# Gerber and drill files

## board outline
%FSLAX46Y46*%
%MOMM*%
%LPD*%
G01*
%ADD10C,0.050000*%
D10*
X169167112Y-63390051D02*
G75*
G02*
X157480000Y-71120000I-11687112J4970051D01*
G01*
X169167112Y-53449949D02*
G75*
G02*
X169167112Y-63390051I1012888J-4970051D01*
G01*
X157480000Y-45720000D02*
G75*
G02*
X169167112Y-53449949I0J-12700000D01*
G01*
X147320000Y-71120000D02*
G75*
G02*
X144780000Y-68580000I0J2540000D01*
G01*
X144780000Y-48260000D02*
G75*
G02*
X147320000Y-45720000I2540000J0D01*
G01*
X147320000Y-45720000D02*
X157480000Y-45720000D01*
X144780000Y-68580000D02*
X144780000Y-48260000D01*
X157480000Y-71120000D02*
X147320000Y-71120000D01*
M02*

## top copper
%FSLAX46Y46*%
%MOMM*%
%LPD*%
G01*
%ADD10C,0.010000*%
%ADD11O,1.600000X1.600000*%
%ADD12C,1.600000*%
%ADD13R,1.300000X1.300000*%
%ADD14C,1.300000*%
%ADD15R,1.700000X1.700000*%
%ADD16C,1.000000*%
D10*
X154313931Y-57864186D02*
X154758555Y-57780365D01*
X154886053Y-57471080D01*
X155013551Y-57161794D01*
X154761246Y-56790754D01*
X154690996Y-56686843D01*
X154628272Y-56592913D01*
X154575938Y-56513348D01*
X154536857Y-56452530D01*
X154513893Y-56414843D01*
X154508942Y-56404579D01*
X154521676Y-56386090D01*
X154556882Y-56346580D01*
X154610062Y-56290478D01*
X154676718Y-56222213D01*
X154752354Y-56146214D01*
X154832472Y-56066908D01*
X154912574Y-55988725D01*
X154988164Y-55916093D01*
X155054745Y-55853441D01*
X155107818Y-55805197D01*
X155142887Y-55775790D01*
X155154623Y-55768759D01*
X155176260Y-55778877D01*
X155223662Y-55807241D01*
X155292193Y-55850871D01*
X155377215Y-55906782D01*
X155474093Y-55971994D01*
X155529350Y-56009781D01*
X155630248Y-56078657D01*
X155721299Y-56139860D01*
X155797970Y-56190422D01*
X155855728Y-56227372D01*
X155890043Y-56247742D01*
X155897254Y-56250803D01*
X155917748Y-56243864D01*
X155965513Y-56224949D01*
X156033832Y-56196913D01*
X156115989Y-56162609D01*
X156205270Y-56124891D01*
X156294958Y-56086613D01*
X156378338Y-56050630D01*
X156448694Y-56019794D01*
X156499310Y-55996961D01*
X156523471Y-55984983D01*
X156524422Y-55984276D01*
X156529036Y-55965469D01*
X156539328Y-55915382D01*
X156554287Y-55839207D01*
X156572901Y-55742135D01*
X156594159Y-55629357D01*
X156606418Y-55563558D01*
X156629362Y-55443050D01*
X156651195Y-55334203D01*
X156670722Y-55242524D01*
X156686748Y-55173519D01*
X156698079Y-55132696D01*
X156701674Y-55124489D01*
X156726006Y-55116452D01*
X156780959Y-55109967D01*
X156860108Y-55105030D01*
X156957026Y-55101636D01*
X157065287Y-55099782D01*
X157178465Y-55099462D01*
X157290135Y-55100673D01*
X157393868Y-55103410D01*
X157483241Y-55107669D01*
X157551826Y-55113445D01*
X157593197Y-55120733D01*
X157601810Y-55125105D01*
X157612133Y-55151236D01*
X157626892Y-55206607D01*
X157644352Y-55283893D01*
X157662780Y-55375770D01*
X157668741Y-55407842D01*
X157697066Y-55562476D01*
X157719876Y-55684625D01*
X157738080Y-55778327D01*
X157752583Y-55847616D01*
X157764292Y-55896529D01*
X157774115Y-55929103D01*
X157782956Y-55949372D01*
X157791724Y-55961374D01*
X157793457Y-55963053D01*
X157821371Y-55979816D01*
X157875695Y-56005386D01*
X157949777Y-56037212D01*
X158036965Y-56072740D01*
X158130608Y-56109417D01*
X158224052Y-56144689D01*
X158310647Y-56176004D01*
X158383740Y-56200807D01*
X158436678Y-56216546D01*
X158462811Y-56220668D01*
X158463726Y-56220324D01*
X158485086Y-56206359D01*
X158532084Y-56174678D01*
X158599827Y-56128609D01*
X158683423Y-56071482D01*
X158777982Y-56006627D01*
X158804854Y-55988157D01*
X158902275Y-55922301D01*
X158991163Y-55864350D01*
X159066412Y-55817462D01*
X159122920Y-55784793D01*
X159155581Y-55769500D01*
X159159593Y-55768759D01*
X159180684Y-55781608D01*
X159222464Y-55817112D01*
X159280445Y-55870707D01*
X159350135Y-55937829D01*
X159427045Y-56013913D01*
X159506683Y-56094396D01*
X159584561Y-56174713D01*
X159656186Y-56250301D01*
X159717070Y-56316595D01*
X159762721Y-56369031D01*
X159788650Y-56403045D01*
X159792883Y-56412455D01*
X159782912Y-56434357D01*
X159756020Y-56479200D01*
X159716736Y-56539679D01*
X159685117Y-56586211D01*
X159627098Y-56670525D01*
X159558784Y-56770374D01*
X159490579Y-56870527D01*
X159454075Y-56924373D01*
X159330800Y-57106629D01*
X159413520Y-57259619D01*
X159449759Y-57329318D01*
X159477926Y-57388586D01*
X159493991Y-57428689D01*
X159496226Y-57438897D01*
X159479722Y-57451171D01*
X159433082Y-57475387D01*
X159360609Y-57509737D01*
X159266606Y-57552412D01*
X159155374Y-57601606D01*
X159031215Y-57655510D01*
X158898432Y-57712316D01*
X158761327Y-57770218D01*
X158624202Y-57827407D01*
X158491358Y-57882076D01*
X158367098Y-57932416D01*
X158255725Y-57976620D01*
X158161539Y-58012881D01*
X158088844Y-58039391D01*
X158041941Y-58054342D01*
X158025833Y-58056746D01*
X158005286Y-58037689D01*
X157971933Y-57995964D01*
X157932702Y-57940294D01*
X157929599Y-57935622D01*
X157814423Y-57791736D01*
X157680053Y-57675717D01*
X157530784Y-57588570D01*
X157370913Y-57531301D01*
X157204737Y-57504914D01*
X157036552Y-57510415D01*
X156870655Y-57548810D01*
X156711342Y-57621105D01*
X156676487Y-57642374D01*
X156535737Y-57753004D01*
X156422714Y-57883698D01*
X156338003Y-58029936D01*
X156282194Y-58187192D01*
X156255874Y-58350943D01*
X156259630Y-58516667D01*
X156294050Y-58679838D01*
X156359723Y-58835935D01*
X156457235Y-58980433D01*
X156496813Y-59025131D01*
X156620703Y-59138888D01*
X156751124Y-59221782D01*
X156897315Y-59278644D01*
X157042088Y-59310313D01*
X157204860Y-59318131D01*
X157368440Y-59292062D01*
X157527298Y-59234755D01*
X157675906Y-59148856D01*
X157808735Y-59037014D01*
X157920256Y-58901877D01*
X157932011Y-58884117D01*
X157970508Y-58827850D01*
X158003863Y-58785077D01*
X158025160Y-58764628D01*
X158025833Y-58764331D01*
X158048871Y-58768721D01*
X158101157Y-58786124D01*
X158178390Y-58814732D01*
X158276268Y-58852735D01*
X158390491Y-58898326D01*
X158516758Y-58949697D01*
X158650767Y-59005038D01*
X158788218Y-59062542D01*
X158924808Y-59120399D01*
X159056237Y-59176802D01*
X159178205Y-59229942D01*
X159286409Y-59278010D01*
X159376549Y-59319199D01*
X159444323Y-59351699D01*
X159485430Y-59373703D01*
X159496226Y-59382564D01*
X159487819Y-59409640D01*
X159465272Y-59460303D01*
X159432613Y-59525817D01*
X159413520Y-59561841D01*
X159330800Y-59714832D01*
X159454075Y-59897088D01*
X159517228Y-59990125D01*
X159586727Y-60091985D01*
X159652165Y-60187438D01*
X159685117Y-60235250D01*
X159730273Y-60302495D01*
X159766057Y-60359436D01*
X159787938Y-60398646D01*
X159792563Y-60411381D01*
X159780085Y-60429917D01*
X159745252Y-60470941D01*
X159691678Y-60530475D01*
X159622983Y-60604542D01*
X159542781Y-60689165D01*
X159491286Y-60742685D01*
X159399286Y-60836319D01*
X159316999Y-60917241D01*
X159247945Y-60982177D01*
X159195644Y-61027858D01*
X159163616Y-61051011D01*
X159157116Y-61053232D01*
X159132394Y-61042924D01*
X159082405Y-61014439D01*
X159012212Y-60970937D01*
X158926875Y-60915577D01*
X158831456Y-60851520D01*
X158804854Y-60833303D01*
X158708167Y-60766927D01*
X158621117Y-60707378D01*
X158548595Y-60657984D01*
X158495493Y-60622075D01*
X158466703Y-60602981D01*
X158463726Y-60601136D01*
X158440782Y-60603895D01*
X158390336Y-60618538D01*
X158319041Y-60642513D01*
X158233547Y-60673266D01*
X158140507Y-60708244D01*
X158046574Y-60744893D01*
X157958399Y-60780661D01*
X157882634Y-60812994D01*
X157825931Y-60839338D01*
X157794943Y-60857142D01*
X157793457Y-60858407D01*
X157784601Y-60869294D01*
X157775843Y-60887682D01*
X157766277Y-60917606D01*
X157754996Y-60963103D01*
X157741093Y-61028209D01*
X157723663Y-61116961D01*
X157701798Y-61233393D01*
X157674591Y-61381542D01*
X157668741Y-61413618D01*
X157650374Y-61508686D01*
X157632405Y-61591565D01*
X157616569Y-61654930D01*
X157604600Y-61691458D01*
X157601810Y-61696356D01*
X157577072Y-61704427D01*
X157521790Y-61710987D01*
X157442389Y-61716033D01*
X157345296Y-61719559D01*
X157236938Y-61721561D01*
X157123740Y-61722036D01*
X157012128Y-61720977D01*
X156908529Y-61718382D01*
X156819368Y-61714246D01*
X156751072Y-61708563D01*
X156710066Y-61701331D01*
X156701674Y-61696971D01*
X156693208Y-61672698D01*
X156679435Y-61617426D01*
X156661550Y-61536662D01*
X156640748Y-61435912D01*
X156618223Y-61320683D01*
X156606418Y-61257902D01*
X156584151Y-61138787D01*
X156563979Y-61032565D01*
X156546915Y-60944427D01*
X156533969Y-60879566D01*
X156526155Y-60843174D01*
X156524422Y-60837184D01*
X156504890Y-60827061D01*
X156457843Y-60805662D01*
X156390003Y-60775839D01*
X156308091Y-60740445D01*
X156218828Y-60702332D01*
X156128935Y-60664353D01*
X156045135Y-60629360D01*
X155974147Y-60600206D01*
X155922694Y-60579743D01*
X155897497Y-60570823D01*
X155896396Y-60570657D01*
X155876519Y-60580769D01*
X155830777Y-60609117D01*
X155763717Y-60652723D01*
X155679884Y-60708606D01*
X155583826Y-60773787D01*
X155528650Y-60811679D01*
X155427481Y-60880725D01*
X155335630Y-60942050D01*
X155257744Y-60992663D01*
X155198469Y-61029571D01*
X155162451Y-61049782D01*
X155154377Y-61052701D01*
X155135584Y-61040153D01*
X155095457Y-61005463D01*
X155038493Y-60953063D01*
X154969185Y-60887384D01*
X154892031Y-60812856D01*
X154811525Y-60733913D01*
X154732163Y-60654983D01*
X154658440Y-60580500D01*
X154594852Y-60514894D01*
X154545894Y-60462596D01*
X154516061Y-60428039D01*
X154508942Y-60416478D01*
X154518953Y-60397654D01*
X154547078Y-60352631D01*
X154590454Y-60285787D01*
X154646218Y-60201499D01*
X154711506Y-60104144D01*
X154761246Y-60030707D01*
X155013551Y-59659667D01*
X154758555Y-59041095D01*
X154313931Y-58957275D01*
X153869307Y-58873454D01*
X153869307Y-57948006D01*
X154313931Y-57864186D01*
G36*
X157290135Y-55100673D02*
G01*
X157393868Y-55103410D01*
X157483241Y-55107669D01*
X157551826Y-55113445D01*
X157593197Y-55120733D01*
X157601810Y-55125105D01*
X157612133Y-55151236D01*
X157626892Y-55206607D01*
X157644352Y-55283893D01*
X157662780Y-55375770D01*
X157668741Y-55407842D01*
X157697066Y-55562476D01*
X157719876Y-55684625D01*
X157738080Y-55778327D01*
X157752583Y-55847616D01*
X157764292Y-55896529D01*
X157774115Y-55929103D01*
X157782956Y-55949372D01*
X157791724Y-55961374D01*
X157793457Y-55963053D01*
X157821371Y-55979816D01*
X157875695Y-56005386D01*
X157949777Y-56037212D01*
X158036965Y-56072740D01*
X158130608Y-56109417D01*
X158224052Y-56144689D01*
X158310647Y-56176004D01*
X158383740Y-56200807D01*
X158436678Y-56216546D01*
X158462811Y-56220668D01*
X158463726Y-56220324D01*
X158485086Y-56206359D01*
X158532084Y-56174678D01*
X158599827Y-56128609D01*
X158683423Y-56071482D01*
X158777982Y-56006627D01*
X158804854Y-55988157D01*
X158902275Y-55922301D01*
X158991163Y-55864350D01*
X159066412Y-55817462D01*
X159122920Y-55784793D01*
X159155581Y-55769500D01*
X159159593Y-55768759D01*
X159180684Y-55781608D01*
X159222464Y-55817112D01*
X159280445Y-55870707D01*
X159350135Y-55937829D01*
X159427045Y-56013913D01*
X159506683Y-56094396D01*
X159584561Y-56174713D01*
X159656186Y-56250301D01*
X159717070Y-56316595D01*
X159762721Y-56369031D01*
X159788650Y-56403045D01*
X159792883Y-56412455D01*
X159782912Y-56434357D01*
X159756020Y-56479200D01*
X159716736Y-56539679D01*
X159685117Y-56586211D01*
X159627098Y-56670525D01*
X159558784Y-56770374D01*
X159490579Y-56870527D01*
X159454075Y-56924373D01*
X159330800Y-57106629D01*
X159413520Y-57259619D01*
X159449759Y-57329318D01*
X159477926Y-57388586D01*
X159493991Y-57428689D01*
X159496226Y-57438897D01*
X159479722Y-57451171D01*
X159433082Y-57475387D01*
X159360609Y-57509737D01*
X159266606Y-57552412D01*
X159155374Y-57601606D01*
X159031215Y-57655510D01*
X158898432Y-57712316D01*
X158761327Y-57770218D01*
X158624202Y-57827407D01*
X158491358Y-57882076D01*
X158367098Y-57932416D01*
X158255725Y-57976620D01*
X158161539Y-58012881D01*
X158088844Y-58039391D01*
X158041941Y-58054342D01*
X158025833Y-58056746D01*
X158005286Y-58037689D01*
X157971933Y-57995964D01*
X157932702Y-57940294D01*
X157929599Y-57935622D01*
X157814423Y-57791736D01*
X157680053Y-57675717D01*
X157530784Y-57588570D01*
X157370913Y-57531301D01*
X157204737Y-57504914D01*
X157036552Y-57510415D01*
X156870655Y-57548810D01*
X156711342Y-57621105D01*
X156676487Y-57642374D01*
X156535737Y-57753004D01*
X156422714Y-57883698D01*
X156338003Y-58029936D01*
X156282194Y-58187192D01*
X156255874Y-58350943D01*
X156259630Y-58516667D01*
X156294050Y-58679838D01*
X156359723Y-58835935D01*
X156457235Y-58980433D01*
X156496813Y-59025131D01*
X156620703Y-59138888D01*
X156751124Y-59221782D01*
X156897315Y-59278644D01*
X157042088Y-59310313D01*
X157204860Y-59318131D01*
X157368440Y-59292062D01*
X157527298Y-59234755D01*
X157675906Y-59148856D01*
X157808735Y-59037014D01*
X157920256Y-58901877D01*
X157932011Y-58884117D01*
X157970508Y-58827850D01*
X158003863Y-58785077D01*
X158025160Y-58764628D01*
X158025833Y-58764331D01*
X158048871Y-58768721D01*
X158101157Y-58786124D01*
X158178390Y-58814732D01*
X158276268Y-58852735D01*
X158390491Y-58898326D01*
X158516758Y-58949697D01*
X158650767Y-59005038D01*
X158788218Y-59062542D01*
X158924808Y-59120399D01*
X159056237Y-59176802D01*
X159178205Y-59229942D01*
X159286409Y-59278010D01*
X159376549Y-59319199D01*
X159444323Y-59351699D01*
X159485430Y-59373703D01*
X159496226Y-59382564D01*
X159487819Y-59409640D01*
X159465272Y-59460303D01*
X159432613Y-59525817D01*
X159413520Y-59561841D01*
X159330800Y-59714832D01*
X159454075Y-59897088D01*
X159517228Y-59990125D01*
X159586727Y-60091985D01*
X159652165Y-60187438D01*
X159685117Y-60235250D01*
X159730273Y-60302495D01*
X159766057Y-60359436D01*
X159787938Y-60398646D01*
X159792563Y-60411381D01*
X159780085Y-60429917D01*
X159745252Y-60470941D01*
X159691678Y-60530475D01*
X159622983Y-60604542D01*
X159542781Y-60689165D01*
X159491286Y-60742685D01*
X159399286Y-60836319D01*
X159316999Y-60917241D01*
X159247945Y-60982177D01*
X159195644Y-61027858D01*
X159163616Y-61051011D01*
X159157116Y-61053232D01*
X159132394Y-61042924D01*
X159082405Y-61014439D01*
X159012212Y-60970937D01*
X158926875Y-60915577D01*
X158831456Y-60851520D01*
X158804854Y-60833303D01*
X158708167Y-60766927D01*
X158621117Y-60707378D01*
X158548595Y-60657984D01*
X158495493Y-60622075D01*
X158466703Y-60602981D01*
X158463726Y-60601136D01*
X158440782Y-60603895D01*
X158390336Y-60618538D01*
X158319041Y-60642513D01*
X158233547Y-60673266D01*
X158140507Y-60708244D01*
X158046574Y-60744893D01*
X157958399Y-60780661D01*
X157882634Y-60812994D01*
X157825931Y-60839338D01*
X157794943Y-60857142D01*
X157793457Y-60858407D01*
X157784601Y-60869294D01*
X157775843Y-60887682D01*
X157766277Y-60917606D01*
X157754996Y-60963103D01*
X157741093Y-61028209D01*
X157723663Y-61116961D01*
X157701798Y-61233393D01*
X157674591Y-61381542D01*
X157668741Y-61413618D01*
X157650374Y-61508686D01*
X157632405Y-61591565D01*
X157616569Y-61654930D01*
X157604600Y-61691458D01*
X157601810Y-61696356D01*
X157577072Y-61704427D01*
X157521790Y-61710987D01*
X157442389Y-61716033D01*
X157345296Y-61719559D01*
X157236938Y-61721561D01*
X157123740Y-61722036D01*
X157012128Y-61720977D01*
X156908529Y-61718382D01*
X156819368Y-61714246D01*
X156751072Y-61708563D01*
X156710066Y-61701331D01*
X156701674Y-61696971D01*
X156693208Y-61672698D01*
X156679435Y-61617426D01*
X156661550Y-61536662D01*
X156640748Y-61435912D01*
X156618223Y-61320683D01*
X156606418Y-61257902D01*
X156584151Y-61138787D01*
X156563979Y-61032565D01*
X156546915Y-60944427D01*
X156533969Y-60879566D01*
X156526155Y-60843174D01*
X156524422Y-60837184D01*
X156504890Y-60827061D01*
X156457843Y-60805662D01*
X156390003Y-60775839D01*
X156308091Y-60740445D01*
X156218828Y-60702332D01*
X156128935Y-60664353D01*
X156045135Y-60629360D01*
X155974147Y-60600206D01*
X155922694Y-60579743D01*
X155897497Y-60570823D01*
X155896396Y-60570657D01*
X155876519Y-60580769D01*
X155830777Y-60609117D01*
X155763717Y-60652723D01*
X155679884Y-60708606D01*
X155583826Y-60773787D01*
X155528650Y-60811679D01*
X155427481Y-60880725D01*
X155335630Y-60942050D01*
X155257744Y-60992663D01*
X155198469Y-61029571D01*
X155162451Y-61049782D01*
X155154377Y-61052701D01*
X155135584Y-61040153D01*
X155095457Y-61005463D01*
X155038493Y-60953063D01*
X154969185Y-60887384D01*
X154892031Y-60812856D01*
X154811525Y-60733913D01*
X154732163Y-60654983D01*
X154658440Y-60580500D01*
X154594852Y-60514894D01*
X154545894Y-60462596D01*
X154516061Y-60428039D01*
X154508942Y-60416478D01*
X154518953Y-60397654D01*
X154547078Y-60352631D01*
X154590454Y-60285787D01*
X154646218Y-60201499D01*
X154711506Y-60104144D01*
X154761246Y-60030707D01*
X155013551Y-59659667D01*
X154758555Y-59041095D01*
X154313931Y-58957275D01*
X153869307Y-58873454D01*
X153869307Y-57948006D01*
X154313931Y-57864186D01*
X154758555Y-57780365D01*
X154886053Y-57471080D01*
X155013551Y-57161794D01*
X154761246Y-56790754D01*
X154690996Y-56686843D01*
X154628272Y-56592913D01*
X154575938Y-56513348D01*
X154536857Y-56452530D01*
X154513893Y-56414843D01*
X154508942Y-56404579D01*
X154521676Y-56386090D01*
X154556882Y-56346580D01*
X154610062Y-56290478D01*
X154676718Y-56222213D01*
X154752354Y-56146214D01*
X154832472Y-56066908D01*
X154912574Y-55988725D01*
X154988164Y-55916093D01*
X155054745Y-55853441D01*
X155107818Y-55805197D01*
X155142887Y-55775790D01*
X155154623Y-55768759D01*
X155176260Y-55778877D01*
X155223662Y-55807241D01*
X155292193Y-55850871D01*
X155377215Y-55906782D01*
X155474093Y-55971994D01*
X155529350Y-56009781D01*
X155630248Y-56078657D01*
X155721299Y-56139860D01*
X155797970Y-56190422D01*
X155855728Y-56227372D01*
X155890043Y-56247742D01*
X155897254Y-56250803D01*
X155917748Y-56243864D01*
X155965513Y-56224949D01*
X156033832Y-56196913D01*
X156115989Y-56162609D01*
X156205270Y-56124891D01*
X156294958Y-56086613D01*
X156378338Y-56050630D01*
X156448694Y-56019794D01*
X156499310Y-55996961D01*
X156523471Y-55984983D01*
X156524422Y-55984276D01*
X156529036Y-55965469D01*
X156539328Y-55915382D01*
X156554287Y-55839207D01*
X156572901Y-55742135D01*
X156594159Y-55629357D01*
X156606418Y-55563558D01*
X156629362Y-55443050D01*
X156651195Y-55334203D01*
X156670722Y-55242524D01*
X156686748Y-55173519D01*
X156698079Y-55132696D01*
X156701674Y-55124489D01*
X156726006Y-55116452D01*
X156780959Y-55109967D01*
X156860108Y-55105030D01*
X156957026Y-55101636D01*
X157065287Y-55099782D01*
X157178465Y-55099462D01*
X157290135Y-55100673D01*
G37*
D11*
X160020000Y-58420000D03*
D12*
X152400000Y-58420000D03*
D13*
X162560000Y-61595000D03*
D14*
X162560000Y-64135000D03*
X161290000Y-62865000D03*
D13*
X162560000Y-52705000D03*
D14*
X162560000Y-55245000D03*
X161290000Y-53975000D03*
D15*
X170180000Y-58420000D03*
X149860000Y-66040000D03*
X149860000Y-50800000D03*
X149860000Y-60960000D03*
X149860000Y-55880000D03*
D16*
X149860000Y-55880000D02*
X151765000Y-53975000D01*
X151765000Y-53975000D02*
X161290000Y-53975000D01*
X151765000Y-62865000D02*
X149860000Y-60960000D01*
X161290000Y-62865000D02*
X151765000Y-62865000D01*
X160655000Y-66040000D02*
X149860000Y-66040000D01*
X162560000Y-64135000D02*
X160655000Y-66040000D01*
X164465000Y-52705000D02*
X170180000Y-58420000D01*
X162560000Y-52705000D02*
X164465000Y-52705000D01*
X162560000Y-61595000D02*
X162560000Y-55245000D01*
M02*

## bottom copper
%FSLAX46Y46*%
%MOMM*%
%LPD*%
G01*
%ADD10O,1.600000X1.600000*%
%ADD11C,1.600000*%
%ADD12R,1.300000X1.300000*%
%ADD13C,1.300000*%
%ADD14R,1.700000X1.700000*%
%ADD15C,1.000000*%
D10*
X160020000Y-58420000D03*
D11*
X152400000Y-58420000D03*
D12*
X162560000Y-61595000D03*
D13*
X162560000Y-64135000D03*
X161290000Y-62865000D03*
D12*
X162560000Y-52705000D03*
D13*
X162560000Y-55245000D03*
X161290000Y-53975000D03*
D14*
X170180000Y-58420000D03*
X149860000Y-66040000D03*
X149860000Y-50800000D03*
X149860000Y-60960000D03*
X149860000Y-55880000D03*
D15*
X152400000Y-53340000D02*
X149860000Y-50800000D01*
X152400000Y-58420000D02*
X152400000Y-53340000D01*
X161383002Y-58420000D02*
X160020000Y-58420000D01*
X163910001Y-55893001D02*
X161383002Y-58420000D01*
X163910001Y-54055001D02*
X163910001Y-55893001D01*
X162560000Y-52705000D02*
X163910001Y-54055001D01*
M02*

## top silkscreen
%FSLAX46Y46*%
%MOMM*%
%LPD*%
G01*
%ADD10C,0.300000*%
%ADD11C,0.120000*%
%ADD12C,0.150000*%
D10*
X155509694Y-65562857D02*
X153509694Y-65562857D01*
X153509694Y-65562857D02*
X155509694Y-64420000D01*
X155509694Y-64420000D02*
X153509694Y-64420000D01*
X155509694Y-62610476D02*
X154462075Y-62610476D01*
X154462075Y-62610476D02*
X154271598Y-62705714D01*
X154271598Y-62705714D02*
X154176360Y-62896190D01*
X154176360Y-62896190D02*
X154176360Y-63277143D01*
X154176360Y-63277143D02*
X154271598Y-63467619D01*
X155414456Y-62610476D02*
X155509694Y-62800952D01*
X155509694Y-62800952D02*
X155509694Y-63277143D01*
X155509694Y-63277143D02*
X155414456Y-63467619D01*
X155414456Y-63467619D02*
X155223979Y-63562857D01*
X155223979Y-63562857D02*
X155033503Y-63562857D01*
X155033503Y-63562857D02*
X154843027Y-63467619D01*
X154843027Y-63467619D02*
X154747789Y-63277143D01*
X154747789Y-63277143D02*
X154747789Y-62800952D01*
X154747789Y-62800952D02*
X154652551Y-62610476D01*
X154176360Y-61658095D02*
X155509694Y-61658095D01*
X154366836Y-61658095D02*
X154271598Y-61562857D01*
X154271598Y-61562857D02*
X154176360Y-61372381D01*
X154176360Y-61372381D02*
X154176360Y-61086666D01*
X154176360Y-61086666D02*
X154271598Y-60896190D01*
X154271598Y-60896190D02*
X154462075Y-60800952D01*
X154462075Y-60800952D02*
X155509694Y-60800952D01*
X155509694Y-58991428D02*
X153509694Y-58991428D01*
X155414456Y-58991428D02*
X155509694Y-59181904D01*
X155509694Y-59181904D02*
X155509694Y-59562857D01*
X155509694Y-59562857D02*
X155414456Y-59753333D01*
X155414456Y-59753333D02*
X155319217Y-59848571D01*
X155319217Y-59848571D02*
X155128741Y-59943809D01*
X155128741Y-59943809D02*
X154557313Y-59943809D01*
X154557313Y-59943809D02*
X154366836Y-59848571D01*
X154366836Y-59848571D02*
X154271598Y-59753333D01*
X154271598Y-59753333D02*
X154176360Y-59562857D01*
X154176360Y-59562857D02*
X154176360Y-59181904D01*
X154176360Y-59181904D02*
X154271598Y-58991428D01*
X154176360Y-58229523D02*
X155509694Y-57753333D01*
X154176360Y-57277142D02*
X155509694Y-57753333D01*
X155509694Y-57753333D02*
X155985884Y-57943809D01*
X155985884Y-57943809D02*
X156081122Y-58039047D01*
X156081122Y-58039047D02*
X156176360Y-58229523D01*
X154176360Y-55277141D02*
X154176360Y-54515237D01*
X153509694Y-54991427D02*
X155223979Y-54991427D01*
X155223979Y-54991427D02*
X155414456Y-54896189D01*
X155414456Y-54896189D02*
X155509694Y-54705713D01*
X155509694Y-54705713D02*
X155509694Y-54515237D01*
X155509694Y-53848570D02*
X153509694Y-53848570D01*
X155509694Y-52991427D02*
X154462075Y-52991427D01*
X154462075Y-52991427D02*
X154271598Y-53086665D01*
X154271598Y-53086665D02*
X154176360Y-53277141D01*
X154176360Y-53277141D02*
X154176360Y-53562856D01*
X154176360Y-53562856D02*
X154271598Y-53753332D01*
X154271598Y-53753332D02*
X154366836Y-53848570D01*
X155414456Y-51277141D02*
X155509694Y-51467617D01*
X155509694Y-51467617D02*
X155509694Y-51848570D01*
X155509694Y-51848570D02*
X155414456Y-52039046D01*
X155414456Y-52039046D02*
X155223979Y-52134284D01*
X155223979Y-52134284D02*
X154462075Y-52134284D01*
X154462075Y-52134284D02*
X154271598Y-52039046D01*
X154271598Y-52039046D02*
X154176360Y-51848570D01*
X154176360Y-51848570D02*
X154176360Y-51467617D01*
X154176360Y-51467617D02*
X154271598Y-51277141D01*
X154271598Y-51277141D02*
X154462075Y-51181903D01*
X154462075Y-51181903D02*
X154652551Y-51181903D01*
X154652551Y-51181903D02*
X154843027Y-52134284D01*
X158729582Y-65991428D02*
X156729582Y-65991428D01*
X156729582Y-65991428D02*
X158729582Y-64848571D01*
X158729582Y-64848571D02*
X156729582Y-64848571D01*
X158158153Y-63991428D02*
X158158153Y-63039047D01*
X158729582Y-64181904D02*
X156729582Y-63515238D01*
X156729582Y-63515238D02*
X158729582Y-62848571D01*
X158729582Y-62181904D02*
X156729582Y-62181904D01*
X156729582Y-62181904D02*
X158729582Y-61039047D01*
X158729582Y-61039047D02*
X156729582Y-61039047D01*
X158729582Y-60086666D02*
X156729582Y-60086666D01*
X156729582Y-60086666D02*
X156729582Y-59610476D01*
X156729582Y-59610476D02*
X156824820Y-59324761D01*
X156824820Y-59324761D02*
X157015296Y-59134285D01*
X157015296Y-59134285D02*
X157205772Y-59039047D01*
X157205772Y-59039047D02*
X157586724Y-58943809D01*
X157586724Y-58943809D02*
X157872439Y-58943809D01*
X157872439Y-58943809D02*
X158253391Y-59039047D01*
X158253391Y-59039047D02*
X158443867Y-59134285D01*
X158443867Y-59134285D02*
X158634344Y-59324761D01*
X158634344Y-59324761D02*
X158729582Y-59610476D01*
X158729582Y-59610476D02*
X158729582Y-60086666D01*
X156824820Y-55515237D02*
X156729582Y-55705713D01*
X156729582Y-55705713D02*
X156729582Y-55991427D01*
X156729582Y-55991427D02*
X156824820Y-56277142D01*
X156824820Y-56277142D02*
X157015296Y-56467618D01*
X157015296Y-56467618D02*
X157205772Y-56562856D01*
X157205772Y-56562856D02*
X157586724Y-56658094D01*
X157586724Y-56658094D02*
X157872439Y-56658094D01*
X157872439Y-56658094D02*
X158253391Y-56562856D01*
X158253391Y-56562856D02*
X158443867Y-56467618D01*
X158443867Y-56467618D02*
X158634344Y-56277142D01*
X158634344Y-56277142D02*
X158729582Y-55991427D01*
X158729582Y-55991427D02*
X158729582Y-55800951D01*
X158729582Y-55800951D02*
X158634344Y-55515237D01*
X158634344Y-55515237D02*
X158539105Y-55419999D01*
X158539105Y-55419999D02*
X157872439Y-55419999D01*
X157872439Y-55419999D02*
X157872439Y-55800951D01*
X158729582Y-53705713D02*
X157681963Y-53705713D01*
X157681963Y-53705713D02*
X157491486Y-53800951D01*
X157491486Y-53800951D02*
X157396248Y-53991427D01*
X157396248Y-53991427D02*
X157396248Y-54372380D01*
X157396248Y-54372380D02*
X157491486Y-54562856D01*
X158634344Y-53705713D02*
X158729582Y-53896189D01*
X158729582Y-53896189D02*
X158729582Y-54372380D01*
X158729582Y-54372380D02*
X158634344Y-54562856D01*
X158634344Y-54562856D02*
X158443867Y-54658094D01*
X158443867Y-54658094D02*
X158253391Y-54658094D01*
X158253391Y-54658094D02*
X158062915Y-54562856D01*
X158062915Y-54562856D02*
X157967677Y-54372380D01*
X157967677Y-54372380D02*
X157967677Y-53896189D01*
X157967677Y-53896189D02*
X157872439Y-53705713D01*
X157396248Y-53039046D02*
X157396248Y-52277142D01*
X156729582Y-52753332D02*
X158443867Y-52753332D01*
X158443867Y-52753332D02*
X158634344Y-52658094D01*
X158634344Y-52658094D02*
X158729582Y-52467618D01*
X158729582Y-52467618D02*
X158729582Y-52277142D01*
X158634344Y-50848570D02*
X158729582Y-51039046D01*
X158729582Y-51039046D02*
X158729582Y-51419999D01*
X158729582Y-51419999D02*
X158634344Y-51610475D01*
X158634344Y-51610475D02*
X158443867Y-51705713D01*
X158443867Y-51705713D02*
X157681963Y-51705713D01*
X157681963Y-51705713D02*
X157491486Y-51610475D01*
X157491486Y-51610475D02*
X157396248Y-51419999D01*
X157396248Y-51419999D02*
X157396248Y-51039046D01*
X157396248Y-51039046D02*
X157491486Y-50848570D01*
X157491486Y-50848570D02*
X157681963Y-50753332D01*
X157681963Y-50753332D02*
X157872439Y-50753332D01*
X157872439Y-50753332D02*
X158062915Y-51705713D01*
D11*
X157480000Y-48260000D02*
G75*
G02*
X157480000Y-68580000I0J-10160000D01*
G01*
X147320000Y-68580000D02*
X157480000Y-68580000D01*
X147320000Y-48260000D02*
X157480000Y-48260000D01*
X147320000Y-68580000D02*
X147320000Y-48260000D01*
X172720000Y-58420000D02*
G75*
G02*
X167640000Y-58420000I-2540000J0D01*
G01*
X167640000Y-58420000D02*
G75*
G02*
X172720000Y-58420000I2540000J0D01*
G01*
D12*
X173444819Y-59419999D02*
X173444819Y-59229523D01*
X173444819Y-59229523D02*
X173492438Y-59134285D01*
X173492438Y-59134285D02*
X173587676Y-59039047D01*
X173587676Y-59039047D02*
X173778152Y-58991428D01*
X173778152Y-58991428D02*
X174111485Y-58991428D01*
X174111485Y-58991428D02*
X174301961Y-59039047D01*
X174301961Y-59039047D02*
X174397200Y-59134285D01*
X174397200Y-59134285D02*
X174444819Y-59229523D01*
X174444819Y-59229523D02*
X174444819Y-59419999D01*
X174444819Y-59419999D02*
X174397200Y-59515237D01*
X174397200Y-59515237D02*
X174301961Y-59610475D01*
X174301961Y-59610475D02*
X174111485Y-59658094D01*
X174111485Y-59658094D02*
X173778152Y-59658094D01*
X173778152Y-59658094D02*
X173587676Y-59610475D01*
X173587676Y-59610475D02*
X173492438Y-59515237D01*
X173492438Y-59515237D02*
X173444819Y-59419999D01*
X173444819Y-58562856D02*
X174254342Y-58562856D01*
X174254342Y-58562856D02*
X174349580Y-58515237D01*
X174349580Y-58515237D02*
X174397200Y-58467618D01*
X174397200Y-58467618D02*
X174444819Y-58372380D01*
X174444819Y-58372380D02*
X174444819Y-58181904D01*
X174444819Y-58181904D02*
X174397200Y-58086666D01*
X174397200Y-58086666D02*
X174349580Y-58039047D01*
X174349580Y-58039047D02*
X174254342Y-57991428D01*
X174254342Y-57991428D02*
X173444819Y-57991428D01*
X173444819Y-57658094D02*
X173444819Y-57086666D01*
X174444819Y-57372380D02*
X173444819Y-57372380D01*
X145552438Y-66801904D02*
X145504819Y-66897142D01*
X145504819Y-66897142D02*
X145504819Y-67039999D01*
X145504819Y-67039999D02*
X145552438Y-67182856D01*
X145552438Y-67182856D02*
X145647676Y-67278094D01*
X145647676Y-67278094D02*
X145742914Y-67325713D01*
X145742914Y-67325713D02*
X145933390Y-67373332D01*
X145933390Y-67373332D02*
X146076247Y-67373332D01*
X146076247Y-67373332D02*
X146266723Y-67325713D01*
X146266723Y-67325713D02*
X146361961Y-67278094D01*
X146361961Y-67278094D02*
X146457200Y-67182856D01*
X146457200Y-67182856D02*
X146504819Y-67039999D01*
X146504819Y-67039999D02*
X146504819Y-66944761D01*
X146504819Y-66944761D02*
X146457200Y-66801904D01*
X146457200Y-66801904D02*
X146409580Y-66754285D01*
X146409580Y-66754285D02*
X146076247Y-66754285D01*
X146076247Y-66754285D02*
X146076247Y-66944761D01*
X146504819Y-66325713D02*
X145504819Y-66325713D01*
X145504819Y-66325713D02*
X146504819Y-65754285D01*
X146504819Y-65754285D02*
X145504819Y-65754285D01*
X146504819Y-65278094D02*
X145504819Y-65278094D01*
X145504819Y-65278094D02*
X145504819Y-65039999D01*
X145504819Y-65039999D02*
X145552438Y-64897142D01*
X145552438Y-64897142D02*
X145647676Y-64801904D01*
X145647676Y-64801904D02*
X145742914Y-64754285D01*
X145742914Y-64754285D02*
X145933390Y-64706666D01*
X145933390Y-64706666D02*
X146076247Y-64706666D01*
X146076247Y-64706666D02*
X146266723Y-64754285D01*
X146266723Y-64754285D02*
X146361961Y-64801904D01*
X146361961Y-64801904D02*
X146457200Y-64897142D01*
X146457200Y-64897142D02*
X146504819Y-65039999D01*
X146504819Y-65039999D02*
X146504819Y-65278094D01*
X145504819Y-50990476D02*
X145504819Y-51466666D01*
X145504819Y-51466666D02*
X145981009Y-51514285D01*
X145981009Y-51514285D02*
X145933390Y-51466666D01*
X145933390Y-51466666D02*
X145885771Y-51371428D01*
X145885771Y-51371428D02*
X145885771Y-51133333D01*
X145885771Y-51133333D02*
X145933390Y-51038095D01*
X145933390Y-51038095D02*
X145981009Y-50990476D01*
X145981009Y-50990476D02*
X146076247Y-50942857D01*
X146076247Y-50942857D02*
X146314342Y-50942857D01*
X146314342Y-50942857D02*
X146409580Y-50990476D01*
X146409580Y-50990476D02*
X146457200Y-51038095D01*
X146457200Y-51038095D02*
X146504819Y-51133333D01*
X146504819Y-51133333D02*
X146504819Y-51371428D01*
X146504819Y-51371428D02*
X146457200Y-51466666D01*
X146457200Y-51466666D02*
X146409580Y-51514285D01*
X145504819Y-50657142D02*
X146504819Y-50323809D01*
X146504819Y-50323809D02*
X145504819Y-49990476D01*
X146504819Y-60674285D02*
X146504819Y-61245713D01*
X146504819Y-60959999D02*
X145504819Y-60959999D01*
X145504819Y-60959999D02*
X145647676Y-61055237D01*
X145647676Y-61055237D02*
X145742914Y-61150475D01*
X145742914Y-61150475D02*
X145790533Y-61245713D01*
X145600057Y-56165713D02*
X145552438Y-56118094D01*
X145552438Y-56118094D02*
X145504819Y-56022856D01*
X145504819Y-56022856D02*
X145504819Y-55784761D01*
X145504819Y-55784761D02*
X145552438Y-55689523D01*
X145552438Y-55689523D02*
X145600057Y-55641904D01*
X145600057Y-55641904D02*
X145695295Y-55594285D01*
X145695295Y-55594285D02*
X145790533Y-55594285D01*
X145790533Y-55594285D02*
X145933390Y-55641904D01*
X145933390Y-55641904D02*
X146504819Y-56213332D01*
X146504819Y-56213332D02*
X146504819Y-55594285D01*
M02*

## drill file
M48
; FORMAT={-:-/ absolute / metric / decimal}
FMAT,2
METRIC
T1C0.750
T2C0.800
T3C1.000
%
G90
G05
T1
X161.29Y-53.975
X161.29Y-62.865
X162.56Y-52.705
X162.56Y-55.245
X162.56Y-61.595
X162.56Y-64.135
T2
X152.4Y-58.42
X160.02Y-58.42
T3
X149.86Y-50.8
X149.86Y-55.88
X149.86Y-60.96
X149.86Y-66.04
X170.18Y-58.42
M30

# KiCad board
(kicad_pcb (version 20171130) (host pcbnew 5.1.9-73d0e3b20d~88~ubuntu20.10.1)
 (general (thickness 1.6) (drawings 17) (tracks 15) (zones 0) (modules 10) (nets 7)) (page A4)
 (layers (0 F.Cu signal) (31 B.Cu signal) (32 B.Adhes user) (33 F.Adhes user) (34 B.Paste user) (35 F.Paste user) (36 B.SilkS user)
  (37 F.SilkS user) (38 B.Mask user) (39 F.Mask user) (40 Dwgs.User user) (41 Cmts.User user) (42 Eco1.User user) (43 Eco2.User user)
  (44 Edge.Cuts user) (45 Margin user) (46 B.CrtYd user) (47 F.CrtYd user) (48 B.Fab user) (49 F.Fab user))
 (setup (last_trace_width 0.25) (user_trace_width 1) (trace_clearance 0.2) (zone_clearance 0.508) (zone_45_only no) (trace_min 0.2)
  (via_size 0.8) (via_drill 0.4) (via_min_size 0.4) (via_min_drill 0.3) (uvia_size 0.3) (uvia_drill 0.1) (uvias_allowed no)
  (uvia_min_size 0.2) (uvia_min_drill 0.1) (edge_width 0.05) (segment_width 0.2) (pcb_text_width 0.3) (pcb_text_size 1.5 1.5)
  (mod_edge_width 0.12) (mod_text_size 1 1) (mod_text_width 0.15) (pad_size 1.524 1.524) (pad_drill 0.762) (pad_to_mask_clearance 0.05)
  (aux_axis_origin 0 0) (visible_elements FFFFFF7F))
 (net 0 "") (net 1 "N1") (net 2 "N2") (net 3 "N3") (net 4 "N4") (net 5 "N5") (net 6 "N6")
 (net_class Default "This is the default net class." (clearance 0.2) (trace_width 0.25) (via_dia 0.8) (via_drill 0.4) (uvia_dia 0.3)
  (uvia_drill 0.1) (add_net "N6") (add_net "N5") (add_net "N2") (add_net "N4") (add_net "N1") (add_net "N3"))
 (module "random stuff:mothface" (layer B.Cu) (at 156.21 66.167 180)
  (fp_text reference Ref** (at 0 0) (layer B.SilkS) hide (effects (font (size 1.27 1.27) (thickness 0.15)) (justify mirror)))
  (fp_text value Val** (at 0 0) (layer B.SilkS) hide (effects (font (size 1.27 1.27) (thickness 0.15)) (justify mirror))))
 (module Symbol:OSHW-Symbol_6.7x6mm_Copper (layer F.Cu) (at 156.845 58.42 90)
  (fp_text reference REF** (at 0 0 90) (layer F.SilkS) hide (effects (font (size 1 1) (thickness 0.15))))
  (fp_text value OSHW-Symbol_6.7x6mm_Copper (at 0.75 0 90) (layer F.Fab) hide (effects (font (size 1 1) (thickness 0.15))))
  (fp_poly
   (pts (xy 0.555814 -2.531069) (xy 0.639635 -2.086445) (xy 0.94892 -1.958947) (xy 1.258206 -1.831449) (xy 1.629246 -2.083754)
    (xy 1.733157 -2.154004) (xy 1.827087 -2.216728) (xy 1.906652 -2.269062) (xy 1.96747 -2.308143) (xy 2.005157 -2.331107)
    (xy 2.015421 -2.336058) (xy 2.03391 -2.323324) (xy 2.07342 -2.288118) (xy 2.129522 -2.234938) (xy 2.197787 -2.168282)
    (xy 2.273786 -2.092646) (xy 2.353092 -2.012528) (xy 2.431275 -1.932426) (xy 2.503907 -1.856836) (xy 2.566559 -1.790255)
    (xy 2.614803 -1.737182) (xy 2.64421 -1.702113) (xy 2.651241 -1.690377) (xy 2.641123 -1.66874) (xy 2.612759 -1.621338)
    (xy 2.569129 -1.552807) (xy 2.513218 -1.467785) (xy 2.448006 -1.370907) (xy 2.410219 -1.31565) (xy 2.341343 -1.214752)
    (xy 2.28014 -1.123701) (xy 2.229578 -1.04703) (xy 2.192628 -0.989272) (xy 2.172258 -0.954957) (xy 2.169197 -0.947746)
    (xy 2.176136 -0.927252) (xy 2.195051 -0.879487) (xy 2.223087 -0.811168) (xy 2.257391 -0.729011) (xy 2.295109 -0.63973)
    (xy 2.333387 -0.550042) (xy 2.36937 -0.466662) (xy 2.400206 -0.396306) (xy 2.423039 -0.34569) (xy 2.435017 -0.321529)
    (xy 2.435724 -0.320578) (xy 2.454531 -0.315964) (xy 2.504618 -0.305672) (xy 2.580793 -0.290713) (xy 2.677865 -0.272099)
    (xy 2.790643 -0.250841) (xy 2.856442 -0.238582) (xy 2.97695 -0.215638) (xy 3.085797 -0.193805) (xy 3.177476 -0.174278)
    (xy 3.246481 -0.158252) (xy 3.287304 -0.146921) (xy 3.295511 -0.143326) (xy 3.303548 -0.118994) (xy 3.310033 -0.064041)
    (xy 3.31497 0.015108) (xy 3.318364 0.112026) (xy 3.320218 0.220287) (xy 3.320538 0.333465) (xy 3.319327 0.445135) (xy 3.31659 0.548868)
    (xy 3.312331 0.638241) (xy 3.306555 0.706826) (xy 3.299267 0.748197) (xy 3.294895 0.75681) (xy 3.268764 0.767133) (xy 3.213393 0.781892)
    (xy 3.136107 0.799352) (xy 3.04423 0.81778) (xy 3.012158 0.823741) (xy 2.857524 0.852066) (xy 2.735375 0.874876) (xy 2.641673 0.89308)
    (xy 2.572384 0.907583) (xy 2.523471 0.919292) (xy 2.490897 0.929115) (xy 2.470628 0.937956) (xy 2.458626 0.946724)
    (xy 2.456947 0.948457) (xy 2.440184 0.976371) (xy 2.414614 1.030695) (xy 2.382788 1.104777) (xy 2.34726 1.191965) (xy 2.310583 1.285608)
    (xy 2.275311 1.379052) (xy 2.243996 1.465647) (xy 2.219193 1.53874) (xy 2.203454 1.591678) (xy 2.199332 1.617811) (xy 2.199676 1.618726)
    (xy 2.213641 1.640086) (xy 2.245322 1.687084) (xy 2.291391 1.754827) (xy 2.348518 1.838423) (xy 2.413373 1.932982)
    (xy 2.431843 1.959854) (xy 2.497699 2.057275) (xy 2.55565 2.146163) (xy 2.602538 2.221412) (xy 2.635207 2.27792) (xy 2.6505 2.310581)
    (xy 2.651241 2.314593) (xy 2.638392 2.335684) (xy 2.602888 2.377464) (xy 2.549293 2.435445) (xy 2.482171 2.505135)
    (xy 2.406087 2.582045) (xy 2.325604 2.661683) (xy 2.245287 2.739561) (xy 2.169699 2.811186) (xy 2.103405 2.87207) (xy 2.050969 2.917721)
    (xy 2.016955 2.94365) (xy 2.007545 2.947883) (xy 1.985643 2.937912) (xy 1.9408 2.91102) (xy 1.880321 2.871736) (xy 1.833789 2.840117)
    (xy 1.749475 2.782098) (xy 1.649626 2.713784) (xy 1.549473 2.645579) (xy 1.495627 2.609075) (xy 1.313371 2.4858) (xy 1.160381 2.56852)
    (xy 1.090682 2.604759) (xy 1.031414 2.632926) (xy 0.991311 2.648991) (xy 0.981103 2.651226) (xy 0.968829 2.634722)
    (xy 0.944613 2.588082) (xy 0.910263 2.515609) (xy 0.867588 2.421606) (xy 0.818394 2.310374) (xy 0.76449 2.186215) (xy 0.707684 2.053432)
    (xy 0.649782 1.916327) (xy 0.592593 1.779202) (xy 0.537924 1.646358) (xy 0.487584 1.522098) (xy 0.44338 1.410725) (xy 0.407119 1.316539)
    (xy 0.380609 1.243844) (xy 0.365658 1.196941) (xy 0.363254 1.180833) (xy 0.382311 1.160286) (xy 0.424036 1.126933)
    (xy 0.479706 1.087702) (xy 0.484378 1.084599) (xy 0.628264 0.969423) (xy 0.744283 0.835053) (xy 0.83143 0.685784) (xy 0.888699 0.525913)
    (xy 0.915086 0.359737) (xy 0.909585 0.191552) (xy 0.87119 0.025655) (xy 0.798895 -0.133658) (xy 0.777626 -0.168513)
    (xy 0.666996 -0.309263) (xy 0.536302 -0.422286) (xy 0.390064 -0.506997) (xy 0.232808 -0.562806) (xy 0.069057 -0.589126)
    (xy -0.096667 -0.58537) (xy -0.259838 -0.55095) (xy -0.415935 -0.485277) (xy -0.560433 -0.387765) (xy -0.605131 -0.348187)
    (xy -0.718888 -0.224297) (xy -0.801782 -0.093876) (xy -0.858644 0.052315) (xy -0.890313 0.197088) (xy -0.898131 0.35986)
    (xy -0.872062 0.52344) (xy -0.814755 0.682298) (xy -0.728856 0.830906) (xy -0.617014 0.963735) (xy -0.481877 1.075256)
    (xy -0.464117 1.087011) (xy -0.40785 1.125508) (xy -0.365077 1.158863) (xy -0.344628 1.18016) (xy -0.344331 1.180833)
    (xy -0.348721 1.203871) (xy -0.366124 1.256157) (xy -0.394732 1.33339) (xy -0.432735 1.431268) (xy -0.478326 1.545491)
    (xy -0.529697 1.671758) (xy -0.585038 1.805767) (xy -0.642542 1.943218) (xy -0.700399 2.079808) (xy -0.756802 2.211237)
    (xy -0.809942 2.333205) (xy -0.85801 2.441409) (xy -0.899199 2.531549) (xy -0.931699 2.599323) (xy -0.953703 2.64043)
    (xy -0.962564 2.651226) (xy -0.98964 2.642819) (xy -1.040303 2.620272) (xy -1.105817 2.587613) (xy -1.141841 2.56852)
    (xy -1.294832 2.4858) (xy -1.477088 2.609075) (xy -1.570125 2.672228) (xy -1.671985 2.741727) (xy -1.767438 2.807165)
    (xy -1.81525 2.840117) (xy -1.882495 2.885273) (xy -1.939436 2.921057) (xy -1.978646 2.942938) (xy -1.991381 2.947563)
    (xy -2.009917 2.935085) (xy -2.050941 2.900252) (xy -2.110475 2.846678) (xy -2.184542 2.777983) (xy -2.269165 2.697781)
    (xy -2.322685 2.646286) (xy -2.416319 2.554286) (xy -2.497241 2.471999) (xy -2.562177 2.402945) (xy -2.607858 2.350644)
    (xy -2.631011 2.318616) (xy -2.633232 2.312116) (xy -2.622924 2.287394) (xy -2.594439 2.237405) (xy -2.550937 2.167212)
    (xy -2.495577 2.081875) (xy -2.43152 1.986456) (xy -2.413303 1.959854) (xy -2.346927 1.863167) (xy -2.287378 1.776117)
    (xy -2.237984 1.703595) (xy -2.202075 1.650493) (xy -2.182981 1.621703) (xy -2.181136 1.618726) (xy -2.183895 1.595782)
    (xy -2.198538 1.545336) (xy -2.222513 1.474041) (xy -2.253266 1.388547) (xy -2.288244 1.295507) (xy -2.324893 1.201574)
    (xy -2.360661 1.113399) (xy -2.392994 1.037634) (xy -2.419338 0.980931) (xy -2.437142 0.949943) (xy -2.438407 0.948457)
    (xy -2.449294 0.939601) (xy -2.467682 0.930843) (xy -2.497606 0.921277) (xy -2.543103 0.909996) (xy -2.608209 0.896093)
    (xy -2.696961 0.878663) (xy -2.813393 0.856798) (xy -2.961542 0.829591) (xy -2.993618 0.823741) (xy -3.088686 0.805374)
    (xy -3.171565 0.787405) (xy -3.23493 0.771569) (xy -3.271458 0.7596) (xy -3.276356 0.75681) (xy -3.284427 0.732072)
    (xy -3.290987 0.67679) (xy -3.296033 0.597389) (xy -3.299559 0.500296) (xy -3.301561 0.391938) (xy -3.302036 0.27874)
    (xy -3.300977 0.167128) (xy -3.298382 0.063529) (xy -3.294246 -0.025632) (xy -3.288563 -0.093928) (xy -3.281331 -0.134934)
    (xy -3.276971 -0.143326) (xy -3.252698 -0.151792) (xy -3.197426 -0.165565) (xy -3.116662 -0.18345) (xy -3.015912 -0.204252)
    (xy -2.900683 -0.226777) (xy -2.837902 -0.238582) (xy -2.718787 -0.260849) (xy -2.612565 -0.281021) (xy -2.524427 -0.298085)
    (xy -2.459566 -0.311031) (xy -2.423174 -0.318845) (xy -2.417184 -0.320578) (xy -2.407061 -0.34011) (xy -2.385662 -0.387157)
    (xy -2.355839 -0.454997) (xy -2.320445 -0.536909) (xy -2.282332 -0.626172) (xy -2.244353 -0.716065) (xy -2.20936 -0.799865)
    (xy -2.180206 -0.870853) (xy -2.159743 -0.922306) (xy -2.150823 -0.947503) (xy -2.150657 -0.948604) (xy -2.160769 -0.968481)
    (xy -2.189117 -1.014223) (xy -2.232723 -1.081283) (xy -2.288606 -1.165116) (xy -2.353787 -1.261174) (xy -2.391679 -1.31635)
    (xy -2.460725 -1.417519) (xy -2.52205 -1.50937) (xy -2.572663 -1.587256) (xy -2.609571 -1.646531) (xy -2.629782 -1.682549)
    (xy -2.632701 -1.690623) (xy -2.620153 -1.709416) (xy -2.585463 -1.749543) (xy -2.533063 -1.806507) (xy -2.467384 -1.875815)
    (xy -2.392856 -1.952969) (xy -2.313913 -2.033475) (xy -2.234983 -2.112837) (xy -2.1605 -2.18656) (xy -2.094894 -2.250148)
    (xy -2.042596 -2.299106) (xy -2.008039 -2.328939) (xy -1.996478 -2.336058) (xy -1.977654 -2.326047) (xy -1.932631 -2.297922)
    (xy -1.865787 -2.254546) (xy -1.781499 -2.198782) (xy -1.684144 -2.133494) (xy -1.610707 -2.083754) (xy -1.239667 -1.831449)
    (xy -0.621095 -2.086445) (xy -0.537275 -2.531069) (xy -0.453454 -2.975693) (xy 0.471994 -2.975693) (xy 0.555814 -2.531069))
   (layer F.Cu) (width 0.01)))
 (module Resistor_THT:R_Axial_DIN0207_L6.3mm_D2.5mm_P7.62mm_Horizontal (layer B.Cu) (at 152.4 58.42)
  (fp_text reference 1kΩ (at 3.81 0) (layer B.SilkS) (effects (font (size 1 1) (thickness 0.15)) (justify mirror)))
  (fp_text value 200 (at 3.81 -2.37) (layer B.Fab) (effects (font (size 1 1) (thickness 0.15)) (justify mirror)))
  (pad 2 thru_hole oval (at 7.62 0) (size 1.6 1.6) (drill 0.8) (layers *.Cu *.Mask) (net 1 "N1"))
  (pad 1 thru_hole circle (at 0 0) (size 1.6 1.6) (drill 0.8) (layers *.Cu *.Mask) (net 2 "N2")))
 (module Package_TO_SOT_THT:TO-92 (layer B.Cu) (at 162.56 61.595 270)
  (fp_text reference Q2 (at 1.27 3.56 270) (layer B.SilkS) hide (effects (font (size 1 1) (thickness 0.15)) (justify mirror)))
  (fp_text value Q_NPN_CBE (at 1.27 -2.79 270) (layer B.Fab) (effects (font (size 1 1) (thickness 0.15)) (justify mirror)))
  (pad 1 thru_hole rect (at 0 0 180) (size 1.3 1.3) (drill 0.75) (layers *.Cu *.Mask) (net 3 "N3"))
  (pad 3 thru_hole circle (at 2.54 0 180) (size 1.3 1.3) (drill 0.75) (layers *.Cu *.Mask) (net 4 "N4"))
  (pad 2 thru_hole circle (at 1.27 1.27 180) (size 1.3 1.3) (drill 0.75) (layers *.Cu *.Mask) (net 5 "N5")))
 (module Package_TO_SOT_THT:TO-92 (layer B.Cu) (at 162.56 52.705 270)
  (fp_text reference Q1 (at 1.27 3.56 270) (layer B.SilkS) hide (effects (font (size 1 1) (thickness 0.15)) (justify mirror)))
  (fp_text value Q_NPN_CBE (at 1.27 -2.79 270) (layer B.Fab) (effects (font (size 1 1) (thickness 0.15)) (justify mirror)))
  (pad 1 thru_hole rect (at 0 0 180) (size 1.3 1.3) (drill 0.75) (layers *.Cu *.Mask) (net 1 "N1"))
  (pad 3 thru_hole circle (at 2.54 0 180) (size 1.3 1.3) (drill 0.75) (layers *.Cu *.Mask) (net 3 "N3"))
  (pad 2 thru_hole circle (at 1.27 1.27 180) (size 1.3 1.3) (drill 0.75) (layers *.Cu *.Mask) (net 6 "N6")))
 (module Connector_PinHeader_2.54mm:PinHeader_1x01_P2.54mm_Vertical (layer B.Cu) (at 170.18 58.42)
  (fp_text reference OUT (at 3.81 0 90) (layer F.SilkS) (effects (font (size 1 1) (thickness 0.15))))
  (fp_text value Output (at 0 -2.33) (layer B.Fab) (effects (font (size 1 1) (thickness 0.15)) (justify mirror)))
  (pad 1 thru_hole rect (at 0 0) (size 1.7 1.7) (drill 1) (layers *.Cu *.Mask) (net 1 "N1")))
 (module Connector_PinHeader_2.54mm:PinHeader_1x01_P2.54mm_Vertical (layer B.Cu) (at 149.86 66.04)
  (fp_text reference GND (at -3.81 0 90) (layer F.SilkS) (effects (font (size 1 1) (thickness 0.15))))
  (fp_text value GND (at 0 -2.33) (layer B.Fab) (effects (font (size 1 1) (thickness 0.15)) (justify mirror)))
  (pad 1 thru_hole rect (at 0 0) (size 1.7 1.7) (drill 1) (layers *.Cu *.Mask) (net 4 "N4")))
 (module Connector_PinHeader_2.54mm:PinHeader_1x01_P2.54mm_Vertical (layer B.Cu) (at 149.86 50.8)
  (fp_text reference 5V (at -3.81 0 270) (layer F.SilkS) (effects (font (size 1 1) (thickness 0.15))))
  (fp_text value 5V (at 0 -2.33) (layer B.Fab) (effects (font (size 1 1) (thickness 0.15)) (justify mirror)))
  (pad 1 thru_hole rect (at 0 0) (size 1.7 1.7) (drill 1) (layers *.Cu *.Mask) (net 2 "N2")))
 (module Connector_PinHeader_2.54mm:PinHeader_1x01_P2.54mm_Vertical (layer B.Cu) (at 149.86 60.96)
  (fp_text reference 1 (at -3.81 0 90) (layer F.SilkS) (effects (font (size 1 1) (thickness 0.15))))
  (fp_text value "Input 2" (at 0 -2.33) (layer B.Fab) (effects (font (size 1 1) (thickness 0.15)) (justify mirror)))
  (pad 1 thru_hole rect (at 0 0) (size 1.7 1.7) (drill 1) (layers *.Cu *.Mask) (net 5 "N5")))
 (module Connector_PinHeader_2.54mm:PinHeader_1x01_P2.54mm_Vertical (layer B.Cu) (at 149.86 55.88)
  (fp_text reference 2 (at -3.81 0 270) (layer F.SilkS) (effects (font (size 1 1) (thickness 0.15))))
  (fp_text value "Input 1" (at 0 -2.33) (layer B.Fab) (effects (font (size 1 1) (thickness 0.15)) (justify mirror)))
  (pad 1 thru_hole rect (at 0 0) (size 1.7 1.7) (drill 1) (layers *.Cu *.Mask) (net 6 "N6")))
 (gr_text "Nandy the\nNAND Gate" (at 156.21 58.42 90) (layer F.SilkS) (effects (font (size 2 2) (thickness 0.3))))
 (gr_arc (start 157.48 58.42) (end 157.48 71.12) (angle -66.96193208) (layer Edge.Cuts) (width 0.05))
 (gr_arc (start 170.18 58.42) (end 169.167112 63.390051) (angle -203.0380715) (layer Edge.Cuts) (width 0.05))
 (gr_arc (start 157.48 58.42) (end 157.48 68.58) (angle -180) (layer F.SilkS) (width 0.12))
 (gr_line (start 147.32 68.58) (end 157.48 68.58) (layer F.SilkS) (width 0.12))
 (gr_line (start 147.32 48.26) (end 157.48 48.26) (layer F.SilkS) (width 0.12))
 (gr_line (start 147.32 68.58) (end 147.32 48.26) (layer F.SilkS) (width 0.12))
 (gr_circle (center 170.18 58.42) (end 170.18 55.88) (layer F.SilkS) (width 0.12))
 (gr_arc (start 157.48 58.42) (end 157.48 45.72) (angle 66.96193208) (layer Edge.Cuts) (width 0.05))
 (gr_arc (start 147.32 68.58) (end 144.78 68.58) (angle -90) (layer Edge.Cuts) (width 0.05))
 (gr_arc (start 147.32 48.26) (end 147.32 45.72) (angle -90) (layer Edge.Cuts) (width 0.05))
 (gr_line (start 147.32 45.72) (end 157.48 45.72) (layer Edge.Cuts) (width 0.05))
 (gr_line (start 144.78 68.58) (end 144.78 48.26) (layer Edge.Cuts) (width 0.05))
 (gr_line (start 157.48 71.12) (end 147.32 71.12) (layer Edge.Cuts) (width 0.05))
 (segment (start 149.86 55.88) (end 151.765 53.975) (width 1) (layer F.Cu) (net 6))
 (segment (start 151.765 53.975) (end 161.29 53.975) (width 1) (layer F.Cu) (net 6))
 (segment (start 151.765 62.865) (end 149.86 60.96) (width 1) (layer F.Cu) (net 5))
 (segment (start 161.29 62.865) (end 151.765 62.865) (width 1) (layer F.Cu) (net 5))
 (segment (start 152.4 53.34) (end 149.86 50.8) (width 1) (layer B.Cu) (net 2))
 (segment (start 152.4 58.42) (end 152.4 53.34) (width 1) (layer B.Cu) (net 2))
 (segment (start 160.655 66.04) (end 149.86 66.04) (width 1) (layer F.Cu) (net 4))
 (segment (start 162.56 64.135) (end 160.655 66.04) (width 1) (layer F.Cu) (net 4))
 (segment (start 164.465 52.705) (end 170.18 58.42) (width 1) (layer F.Cu) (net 1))
 (segment (start 162.56 52.705) (end 164.465 52.705) (width 1) (layer F.Cu) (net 1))
 (segment (start 161.383002 58.42) (end 160.02 58.42) (width 1) (layer B.Cu) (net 1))
 (segment (start 163.910001 55.893001) (end 161.383002 58.42) (width 1) (layer B.Cu) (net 1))
 (segment (start 163.910001 54.055001) (end 163.910001 55.893001) (width 1) (layer B.Cu) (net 1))
 (segment (start 162.56 52.705) (end 163.910001 54.055001) (width 1) (layer B.Cu) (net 1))
 (segment (start 162.56 61.595) (end 162.56 55.245) (width 1) (layer F.Cu) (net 3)))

